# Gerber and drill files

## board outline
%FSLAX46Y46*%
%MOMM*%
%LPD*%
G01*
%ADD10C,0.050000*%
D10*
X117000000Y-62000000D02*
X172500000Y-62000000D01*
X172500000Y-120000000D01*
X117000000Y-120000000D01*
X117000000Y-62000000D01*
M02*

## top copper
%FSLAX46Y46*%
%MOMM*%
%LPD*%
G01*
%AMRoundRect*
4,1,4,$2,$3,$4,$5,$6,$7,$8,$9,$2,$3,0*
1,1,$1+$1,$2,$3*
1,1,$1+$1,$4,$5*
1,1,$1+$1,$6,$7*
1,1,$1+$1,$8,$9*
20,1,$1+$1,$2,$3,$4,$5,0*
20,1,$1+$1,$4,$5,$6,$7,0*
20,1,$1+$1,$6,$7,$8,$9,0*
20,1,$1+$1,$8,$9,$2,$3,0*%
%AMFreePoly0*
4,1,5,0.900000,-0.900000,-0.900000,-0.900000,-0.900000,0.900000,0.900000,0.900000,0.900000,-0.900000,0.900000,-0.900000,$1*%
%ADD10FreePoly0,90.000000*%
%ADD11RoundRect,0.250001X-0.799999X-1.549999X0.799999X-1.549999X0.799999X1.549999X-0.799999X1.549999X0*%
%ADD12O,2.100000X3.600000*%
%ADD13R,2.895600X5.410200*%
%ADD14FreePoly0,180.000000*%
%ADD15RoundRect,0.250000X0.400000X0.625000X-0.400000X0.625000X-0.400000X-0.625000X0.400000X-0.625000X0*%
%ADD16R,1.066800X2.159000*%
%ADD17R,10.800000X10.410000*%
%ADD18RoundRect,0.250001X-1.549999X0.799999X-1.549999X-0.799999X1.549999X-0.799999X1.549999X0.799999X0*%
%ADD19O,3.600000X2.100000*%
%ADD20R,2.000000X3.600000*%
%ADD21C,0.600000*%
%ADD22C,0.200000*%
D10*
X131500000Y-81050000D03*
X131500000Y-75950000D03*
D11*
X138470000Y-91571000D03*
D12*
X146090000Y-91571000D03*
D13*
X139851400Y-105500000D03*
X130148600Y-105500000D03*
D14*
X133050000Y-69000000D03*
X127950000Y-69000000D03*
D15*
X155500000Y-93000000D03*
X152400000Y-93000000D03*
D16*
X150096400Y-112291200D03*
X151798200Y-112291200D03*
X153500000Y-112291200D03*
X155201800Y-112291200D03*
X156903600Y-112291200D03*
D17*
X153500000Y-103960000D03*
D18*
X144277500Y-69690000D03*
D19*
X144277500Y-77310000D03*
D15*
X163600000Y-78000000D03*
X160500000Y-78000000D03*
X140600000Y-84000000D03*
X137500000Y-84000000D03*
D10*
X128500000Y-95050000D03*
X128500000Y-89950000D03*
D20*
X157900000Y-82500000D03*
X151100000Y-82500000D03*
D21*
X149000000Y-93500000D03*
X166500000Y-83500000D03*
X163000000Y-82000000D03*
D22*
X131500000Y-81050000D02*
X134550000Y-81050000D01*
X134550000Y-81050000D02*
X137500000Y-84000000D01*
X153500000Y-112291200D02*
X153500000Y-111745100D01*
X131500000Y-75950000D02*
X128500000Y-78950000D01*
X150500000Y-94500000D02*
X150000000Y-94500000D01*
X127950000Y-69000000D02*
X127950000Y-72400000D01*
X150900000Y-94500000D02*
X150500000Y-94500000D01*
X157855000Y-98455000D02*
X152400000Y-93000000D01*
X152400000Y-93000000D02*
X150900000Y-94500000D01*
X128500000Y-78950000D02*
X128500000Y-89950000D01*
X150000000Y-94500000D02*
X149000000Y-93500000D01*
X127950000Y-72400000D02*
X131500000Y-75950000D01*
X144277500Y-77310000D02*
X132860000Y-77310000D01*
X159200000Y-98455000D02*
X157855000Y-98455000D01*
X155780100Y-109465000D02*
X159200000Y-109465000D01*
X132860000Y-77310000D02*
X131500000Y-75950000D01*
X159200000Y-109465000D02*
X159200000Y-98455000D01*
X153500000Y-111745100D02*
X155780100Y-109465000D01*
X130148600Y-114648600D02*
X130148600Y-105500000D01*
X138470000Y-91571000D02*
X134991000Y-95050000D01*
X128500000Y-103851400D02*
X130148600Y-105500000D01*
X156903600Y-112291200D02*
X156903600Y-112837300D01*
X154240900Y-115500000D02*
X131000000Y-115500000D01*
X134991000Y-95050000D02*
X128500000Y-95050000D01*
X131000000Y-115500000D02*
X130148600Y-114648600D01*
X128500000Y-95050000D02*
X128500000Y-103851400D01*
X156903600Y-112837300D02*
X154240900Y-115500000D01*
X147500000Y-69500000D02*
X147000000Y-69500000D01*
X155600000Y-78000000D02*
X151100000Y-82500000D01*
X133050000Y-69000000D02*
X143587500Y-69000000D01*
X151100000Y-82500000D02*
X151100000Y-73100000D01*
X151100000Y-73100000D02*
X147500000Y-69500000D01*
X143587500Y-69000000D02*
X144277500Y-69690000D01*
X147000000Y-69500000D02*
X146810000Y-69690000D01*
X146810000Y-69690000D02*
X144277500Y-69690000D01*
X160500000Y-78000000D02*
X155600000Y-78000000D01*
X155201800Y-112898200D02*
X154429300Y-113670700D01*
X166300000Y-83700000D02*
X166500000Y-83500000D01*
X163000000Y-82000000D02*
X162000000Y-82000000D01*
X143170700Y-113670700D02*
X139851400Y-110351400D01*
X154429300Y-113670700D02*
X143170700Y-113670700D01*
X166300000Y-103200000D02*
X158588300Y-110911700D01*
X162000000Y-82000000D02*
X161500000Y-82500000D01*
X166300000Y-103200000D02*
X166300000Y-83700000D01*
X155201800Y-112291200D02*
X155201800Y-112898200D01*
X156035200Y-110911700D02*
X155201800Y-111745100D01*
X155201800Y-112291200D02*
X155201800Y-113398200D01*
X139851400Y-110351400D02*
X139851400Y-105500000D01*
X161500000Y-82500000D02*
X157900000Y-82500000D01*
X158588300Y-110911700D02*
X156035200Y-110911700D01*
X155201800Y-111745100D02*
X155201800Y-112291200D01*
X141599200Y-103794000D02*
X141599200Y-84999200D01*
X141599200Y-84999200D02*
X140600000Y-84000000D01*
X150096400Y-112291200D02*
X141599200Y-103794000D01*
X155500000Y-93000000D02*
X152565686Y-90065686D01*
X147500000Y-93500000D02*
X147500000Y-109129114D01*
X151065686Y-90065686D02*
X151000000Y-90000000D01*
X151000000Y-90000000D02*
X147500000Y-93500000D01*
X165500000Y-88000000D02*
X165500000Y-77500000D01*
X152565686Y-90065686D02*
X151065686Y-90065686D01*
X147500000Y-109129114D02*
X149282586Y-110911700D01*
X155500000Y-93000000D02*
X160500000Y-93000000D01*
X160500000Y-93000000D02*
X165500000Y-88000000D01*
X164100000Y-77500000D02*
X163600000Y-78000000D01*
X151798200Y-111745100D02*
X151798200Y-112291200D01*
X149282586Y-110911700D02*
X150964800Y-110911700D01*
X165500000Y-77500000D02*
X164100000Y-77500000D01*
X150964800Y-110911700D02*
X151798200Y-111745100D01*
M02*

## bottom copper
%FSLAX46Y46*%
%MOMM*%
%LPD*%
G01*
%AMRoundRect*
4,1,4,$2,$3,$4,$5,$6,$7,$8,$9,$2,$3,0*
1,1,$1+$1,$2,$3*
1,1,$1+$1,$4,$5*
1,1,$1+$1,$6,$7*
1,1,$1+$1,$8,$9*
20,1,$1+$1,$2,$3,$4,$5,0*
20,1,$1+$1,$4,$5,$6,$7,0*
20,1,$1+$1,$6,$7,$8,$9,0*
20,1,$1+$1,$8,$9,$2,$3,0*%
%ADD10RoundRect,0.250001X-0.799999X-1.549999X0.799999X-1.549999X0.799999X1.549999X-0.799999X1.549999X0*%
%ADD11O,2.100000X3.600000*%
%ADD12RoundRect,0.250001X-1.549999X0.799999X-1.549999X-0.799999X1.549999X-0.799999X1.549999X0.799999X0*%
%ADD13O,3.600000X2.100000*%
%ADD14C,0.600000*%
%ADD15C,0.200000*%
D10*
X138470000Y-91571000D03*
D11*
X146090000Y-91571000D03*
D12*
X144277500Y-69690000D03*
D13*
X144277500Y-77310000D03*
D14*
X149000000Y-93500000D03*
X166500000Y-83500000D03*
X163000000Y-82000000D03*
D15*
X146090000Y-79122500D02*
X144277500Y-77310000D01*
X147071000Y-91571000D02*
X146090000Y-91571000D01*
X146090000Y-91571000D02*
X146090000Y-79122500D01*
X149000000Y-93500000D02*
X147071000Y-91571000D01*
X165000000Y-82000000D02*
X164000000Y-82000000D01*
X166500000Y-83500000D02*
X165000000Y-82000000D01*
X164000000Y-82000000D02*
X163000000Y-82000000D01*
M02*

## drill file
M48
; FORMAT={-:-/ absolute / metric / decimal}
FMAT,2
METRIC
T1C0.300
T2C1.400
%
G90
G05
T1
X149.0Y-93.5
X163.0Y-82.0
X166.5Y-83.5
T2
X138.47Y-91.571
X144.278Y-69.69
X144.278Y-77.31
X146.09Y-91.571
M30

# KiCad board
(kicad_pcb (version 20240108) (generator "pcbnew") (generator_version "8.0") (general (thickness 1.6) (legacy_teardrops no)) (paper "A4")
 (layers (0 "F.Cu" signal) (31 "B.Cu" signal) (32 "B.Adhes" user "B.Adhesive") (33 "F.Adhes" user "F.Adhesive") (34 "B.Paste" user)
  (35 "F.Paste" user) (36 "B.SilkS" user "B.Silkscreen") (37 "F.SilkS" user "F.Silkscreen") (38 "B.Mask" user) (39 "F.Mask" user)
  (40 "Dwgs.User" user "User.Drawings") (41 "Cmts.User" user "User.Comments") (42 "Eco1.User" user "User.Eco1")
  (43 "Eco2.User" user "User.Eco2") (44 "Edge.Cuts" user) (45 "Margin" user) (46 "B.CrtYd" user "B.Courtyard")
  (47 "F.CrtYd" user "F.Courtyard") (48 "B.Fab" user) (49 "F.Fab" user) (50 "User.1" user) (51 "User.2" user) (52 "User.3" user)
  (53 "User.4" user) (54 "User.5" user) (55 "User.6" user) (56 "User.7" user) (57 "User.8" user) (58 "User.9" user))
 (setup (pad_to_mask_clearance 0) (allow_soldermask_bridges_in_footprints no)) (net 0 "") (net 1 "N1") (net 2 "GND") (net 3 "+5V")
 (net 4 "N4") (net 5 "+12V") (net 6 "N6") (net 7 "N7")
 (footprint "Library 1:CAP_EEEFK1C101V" (layer "F.Cu") (at 131.5 78.5 90)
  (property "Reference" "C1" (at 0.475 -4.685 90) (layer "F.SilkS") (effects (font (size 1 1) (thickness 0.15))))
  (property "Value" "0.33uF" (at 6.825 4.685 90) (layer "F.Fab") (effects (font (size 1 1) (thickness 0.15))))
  (pad "1" smd custom (at -2.55 0 90) (size 1.8 1.8) (layers "F.Cu") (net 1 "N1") (options (clearance outline) (anchor rect)) (primitives))
  (pad "2" smd custom (at 2.55 0 90) (size 1.8 1.8) (layers "F.Cu") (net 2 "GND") (options (clearance outline) (anchor rect)) (primitives)))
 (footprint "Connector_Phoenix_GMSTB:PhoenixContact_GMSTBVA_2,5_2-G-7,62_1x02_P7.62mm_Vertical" (layer "F.Cu") (at 138.47 91.571)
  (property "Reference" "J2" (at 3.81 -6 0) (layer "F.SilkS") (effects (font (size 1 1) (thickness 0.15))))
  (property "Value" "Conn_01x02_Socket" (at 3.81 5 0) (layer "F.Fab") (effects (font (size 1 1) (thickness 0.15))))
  (pad "1" thru_hole roundrect (at 0 0) (size 2.1 3.6) (drill 1.4) (layers "*.Cu" "*.Mask") (remove_unused_layers no)
   (roundrect_rratio 0.119048) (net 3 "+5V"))
  (pad "2" thru_hole oval (at 7.62 0) (size 2.1 3.6) (drill 1.4) (layers "*.Cu" "*.Mask") (remove_unused_layers no) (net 2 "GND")))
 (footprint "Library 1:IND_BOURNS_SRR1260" (layer "F.Cu") (at 135 105.5 180)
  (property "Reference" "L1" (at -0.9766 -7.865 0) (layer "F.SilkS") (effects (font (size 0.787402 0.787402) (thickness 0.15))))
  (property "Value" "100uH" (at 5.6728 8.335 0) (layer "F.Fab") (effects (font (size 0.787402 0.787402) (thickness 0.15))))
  (pad "1" smd rect (at -4.8514 0 180) (size 2.8956 5.4102) (layers "F.Cu" "F.Paste" "F.Mask") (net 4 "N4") (solder_mask_margin 0.102))
  (pad "2" smd rect (at 4.8514 0 180) (size 2.8956 5.4102) (layers "F.Cu" "F.Paste" "F.Mask") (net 3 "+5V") (solder_mask_margin 0.102)))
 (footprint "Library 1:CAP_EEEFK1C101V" (layer "F.Cu") (at 130.5 69 180)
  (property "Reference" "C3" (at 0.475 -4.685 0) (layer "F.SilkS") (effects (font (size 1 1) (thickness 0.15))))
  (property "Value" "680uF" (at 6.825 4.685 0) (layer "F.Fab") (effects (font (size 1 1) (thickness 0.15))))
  (pad "1" smd custom (at -2.55 0 180) (size 1.8 1.8) (layers "F.Cu") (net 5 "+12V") (options (clearance outline) (anchor rect))
   (primitives))
  (pad "2" smd custom (at 2.55 0 180) (size 1.8 1.8) (layers "F.Cu") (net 2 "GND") (options (clearance outline) (anchor rect)) (primitives)))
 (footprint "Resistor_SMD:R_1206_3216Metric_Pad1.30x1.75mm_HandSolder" (layer "F.Cu") (at 153.95 93 180)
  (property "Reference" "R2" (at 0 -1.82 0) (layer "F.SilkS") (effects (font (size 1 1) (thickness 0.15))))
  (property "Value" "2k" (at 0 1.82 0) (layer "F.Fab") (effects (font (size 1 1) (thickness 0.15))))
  (pad "1" smd roundrect (at -1.55 0 180) (size 1.3 1.75) (layers "F.Cu" "F.Paste" "F.Mask") (roundrect_rratio 0.192308) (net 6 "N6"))
  (pad "2" smd roundrect (at 1.55 0 180) (size 1.3 1.75) (layers "F.Cu" "F.Paste" "F.Mask") (roundrect_rratio 0.192308) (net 2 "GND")))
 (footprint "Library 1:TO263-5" (layer "F.Cu") (at 153.5 106.5)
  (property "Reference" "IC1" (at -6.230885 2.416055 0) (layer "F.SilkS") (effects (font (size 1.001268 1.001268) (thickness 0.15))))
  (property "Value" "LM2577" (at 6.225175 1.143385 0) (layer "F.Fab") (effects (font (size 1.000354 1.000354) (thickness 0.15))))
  (pad "1" smd rect (at -3.4036 5.7912) (size 1.0668 2.159) (layers "F.Cu" "F.Paste" "F.Mask") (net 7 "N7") (solder_mask_margin 0.102))
  (pad "2" smd rect (at -1.7018 5.7912) (size 1.0668 2.159) (layers "F.Cu" "F.Paste" "F.Mask") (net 6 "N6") (solder_mask_margin 0.102))
  (pad "3" smd rect (at 0 5.7912) (size 1.0668 2.159) (layers "F.Cu" "F.Paste" "F.Mask") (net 2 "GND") (solder_mask_margin 0.102))
  (pad "4" smd rect (at 1.7018 5.7912) (size 1.0668 2.159) (layers "F.Cu" "F.Paste" "F.Mask") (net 4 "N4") (solder_mask_margin 0.102))
  (pad "5" smd rect (at 3.4036 5.7912) (size 1.0668 2.159) (layers "F.Cu" "F.Paste" "F.Mask") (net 3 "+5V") (solder_mask_margin 0.102))
  (pad "6" smd rect (at 0 -2.54) (size 10.8 10.41) (layers "F.Cu" "F.Paste" "F.Mask") (solder_mask_margin 0.102)))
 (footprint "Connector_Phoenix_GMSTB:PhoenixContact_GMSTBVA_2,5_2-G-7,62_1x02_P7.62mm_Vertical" (layer "F.Cu") (at 144.2775 69.69 -90)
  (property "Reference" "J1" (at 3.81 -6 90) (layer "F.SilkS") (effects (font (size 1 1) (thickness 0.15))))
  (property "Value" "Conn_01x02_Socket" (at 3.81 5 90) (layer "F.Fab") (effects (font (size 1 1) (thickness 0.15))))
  (pad "1" thru_hole roundrect (at 0 0 270) (size 2.1 3.6) (drill 1.4) (layers "*.Cu" "*.Mask") (remove_unused_layers no)
   (roundrect_rratio 0.119048) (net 5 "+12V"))
  (pad "2" thru_hole oval (at 7.62 0 270) (size 2.1 3.6) (drill 1.4) (layers "*.Cu" "*.Mask") (remove_unused_layers no) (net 2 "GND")))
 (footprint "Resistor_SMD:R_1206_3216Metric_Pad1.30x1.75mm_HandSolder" (layer "F.Cu") (at 162.05 78 180)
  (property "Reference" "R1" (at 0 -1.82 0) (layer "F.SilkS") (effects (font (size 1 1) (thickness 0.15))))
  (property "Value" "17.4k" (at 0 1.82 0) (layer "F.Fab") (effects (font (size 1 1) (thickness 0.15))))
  (pad "1" smd roundrect (at -1.55 0 180) (size 1.3 1.75) (layers "F.Cu" "F.Paste" "F.Mask") (roundrect_rratio 0.192308) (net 6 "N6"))
  (pad "2" smd roundrect (at 1.55 0 180) (size 1.3 1.75) (layers "F.Cu" "F.Paste" "F.Mask") (roundrect_rratio 0.192308) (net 5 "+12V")))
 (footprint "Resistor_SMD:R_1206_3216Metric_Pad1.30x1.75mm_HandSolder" (layer "F.Cu") (at 139.05 84 180)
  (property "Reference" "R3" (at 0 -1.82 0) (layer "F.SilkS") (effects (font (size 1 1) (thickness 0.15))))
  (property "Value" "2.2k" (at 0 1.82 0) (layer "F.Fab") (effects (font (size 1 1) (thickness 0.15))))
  (pad "1" smd roundrect (at -1.55 0 180) (size 1.3 1.75) (layers "F.Cu" "F.Paste" "F.Mask") (roundrect_rratio 0.192308) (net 7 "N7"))
  (pad "2" smd roundrect (at 1.55 0 180) (size 1.3 1.75) (layers "F.Cu" "F.Paste" "F.Mask") (roundrect_rratio 0.192308) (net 1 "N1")))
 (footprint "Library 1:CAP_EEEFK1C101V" (layer "F.Cu") (at 128.5 92.5 90)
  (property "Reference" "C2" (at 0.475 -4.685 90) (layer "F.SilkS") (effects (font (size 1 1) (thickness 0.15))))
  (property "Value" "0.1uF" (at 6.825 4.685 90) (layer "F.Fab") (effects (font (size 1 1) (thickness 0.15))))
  (pad "1" smd custom (at -2.55 0 90) (size 1.8 1.8) (layers "F.Cu") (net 3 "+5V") (options (clearance outline) (anchor rect)) (primitives))
  (pad "2" smd custom (at 2.55 0 90) (size 1.8 1.8) (layers "F.Cu") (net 2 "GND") (options (clearance outline) (anchor rect)) (primitives)))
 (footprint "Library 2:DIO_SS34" (layer "F.Cu") (at 154.5 82.5)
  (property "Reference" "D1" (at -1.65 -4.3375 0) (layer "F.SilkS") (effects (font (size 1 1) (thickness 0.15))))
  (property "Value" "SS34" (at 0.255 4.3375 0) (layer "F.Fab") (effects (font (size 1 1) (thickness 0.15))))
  (pad "A" smd rect (at 3.4 0) (size 2 3.6) (layers "F.Cu" "F.Paste" "F.Mask") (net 4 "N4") (solder_mask_margin 0.102))
  (pad "C" smd rect (at -3.4 0) (size 2 3.6) (layers "F.Cu" "F.Paste" "F.Mask") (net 5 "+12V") (solder_mask_margin 0.102)))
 (gr_rect (start 117 62) (end 172.5 120) (stroke (width 0.05) (type default)) (fill none) (layer "Edge.Cuts"))
 (segment (start 131.5 81.05) (end 134.55 81.05) (width 0.2) (layer "F.Cu") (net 1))
 (segment (start 134.55 81.05) (end 137.5 84) (width 0.2) (layer "F.Cu") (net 1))
 (segment (start 153.5 112.2912) (end 153.5 111.7451) (width 0.2) (layer "F.Cu") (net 2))
 (segment (start 131.5 75.95) (end 128.5 78.95) (width 0.2) (layer "F.Cu") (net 2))
 (segment (start 150.5 94.5) (end 150 94.5) (width 0.2) (layer "F.Cu") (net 2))
 (segment (start 127.95 69) (end 127.95 72.4) (width 0.2) (layer "F.Cu") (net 2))
 (segment (start 150.9 94.5) (end 150.5 94.5) (width 0.2) (layer "F.Cu") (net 2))
 (segment (start 157.855 98.455) (end 152.4 93) (width 0.2) (layer "F.Cu") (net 2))
 (segment (start 152.4 93) (end 150.9 94.5) (width 0.2) (layer "F.Cu") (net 2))
 (segment (start 128.5 78.95) (end 128.5 89.95) (width 0.2) (layer "F.Cu") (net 2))
 (segment (start 150 94.5) (end 149 93.5) (width 0.2) (layer "F.Cu") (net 2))
 (segment (start 127.95 72.4) (end 131.5 75.95) (width 0.2) (layer "F.Cu") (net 2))
 (segment (start 144.2775 77.31) (end 132.86 77.31) (width 0.2) (layer "F.Cu") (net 2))
 (segment (start 159.2 98.455) (end 157.855 98.455) (width 0.2) (layer "F.Cu") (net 2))
 (segment (start 155.7801 109.465) (end 159.2 109.465) (width 0.2) (layer "F.Cu") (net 2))
 (segment (start 132.86 77.31) (end 131.5 75.95) (width 0.2) (layer "F.Cu") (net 2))
 (segment (start 159.2 109.465) (end 159.2 98.455) (width 0.2) (layer "F.Cu") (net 2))
 (segment (start 153.5 111.7451) (end 155.7801 109.465) (width 0.2) (layer "F.Cu") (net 2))
 (via (at 149 93.5) (size 0.6) (drill 0.3) (layers "F.Cu" "B.Cu") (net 2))
 (segment (start 146.09 79.1225) (end 144.2775 77.31) (width 0.2) (layer "B.Cu") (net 2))
 (segment (start 147.071 91.571) (end 146.09 91.571) (width 0.2) (layer "B.Cu") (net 2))
 (segment (start 146.09 91.571) (end 146.09 79.1225) (width 0.2) (layer "B.Cu") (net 2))
 (segment (start 149 93.5) (end 147.071 91.571) (width 0.2) (layer "B.Cu") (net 2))
 (segment (start 130.1486 114.6486) (end 130.1486 105.5) (width 0.2) (layer "F.Cu") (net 3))
 (segment (start 138.47 91.571) (end 134.991 95.05) (width 0.2) (layer "F.Cu") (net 3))
 (segment (start 128.5 103.8514) (end 130.1486 105.5) (width 0.2) (layer "F.Cu") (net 3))
 (segment (start 156.9036 112.2912) (end 156.9036 112.8373) (width 0.2) (layer "F.Cu") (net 3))
 (segment (start 154.2409 115.5) (end 131 115.5) (width 0.2) (layer "F.Cu") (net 3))
 (segment (start 134.991 95.05) (end 128.5 95.05) (width 0.2) (layer "F.Cu") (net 3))
 (segment (start 131 115.5) (end 130.1486 114.6486) (width 0.2) (layer "F.Cu") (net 3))
 (segment (start 128.5 95.05) (end 128.5 103.8514) (width 0.2) (layer "F.Cu") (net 3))
 (segment (start 156.9036 112.8373) (end 154.2409 115.5) (width 0.2) (layer "F.Cu") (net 3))
 (segment (start 147.5 69.5) (end 147 69.5) (width 0.2) (layer "F.Cu") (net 5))
 (segment (start 155.6 78) (end 151.1 82.5) (width 0.2) (layer "F.Cu") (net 5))
 (segment (start 133.05 69) (end 143.5875 69) (width 0.2) (layer "F.Cu") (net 5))
 (segment (start 151.1 82.5) (end 151.1 73.1) (width 0.2) (layer "F.Cu") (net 5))
 (segment (start 151.1 73.1) (end 147.5 69.5) (width 0.2) (layer "F.Cu") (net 5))
 (segment (start 143.5875 69) (end 144.2775 69.69) (width 0.2) (layer "F.Cu") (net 5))
 (segment (start 147 69.5) (end 146.81 69.69) (width 0.2) (layer "F.Cu") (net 5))
 (segment (start 146.81 69.69) (end 144.2775 69.69) (width 0.2) (layer "F.Cu") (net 5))
 (segment (start 160.5 78) (end 155.6 78) (width 0.2) (layer "F.Cu") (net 5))
 (segment (start 155.2018 112.8982) (end 154.4293 113.6707) (width 0.2) (layer "F.Cu") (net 4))
 (segment (start 166.3 83.7) (end 166.5 83.5) (width 0.2) (layer "F.Cu") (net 4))
 (segment (start 163 82) (end 162 82) (width 0.2) (layer "F.Cu") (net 4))
 (segment (start 143.1707 113.6707) (end 139.8514 110.3514) (width 0.2) (layer "F.Cu") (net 4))
 (segment (start 154.4293 113.6707) (end 143.1707 113.6707) (width 0.2) (layer "F.Cu") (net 4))
 (segment (start 166.3 103.2) (end 158.5883 110.9117) (width 0.2) (layer "F.Cu") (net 4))
 (segment (start 162 82) (end 161.5 82.5) (width 0.2) (layer "F.Cu") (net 4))
 (segment (start 166.3 103.2) (end 166.3 83.7) (width 0.2) (layer "F.Cu") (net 4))
 (segment (start 155.2018 112.2912) (end 155.2018 112.8982) (width 0.2) (layer "F.Cu") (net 4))
 (segment (start 156.0352 110.9117) (end 155.2018 111.7451) (width 0.2) (layer "F.Cu") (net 4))
 (segment (start 155.2018 112.2912) (end 155.2018 113.3982) (width 0.2) (layer "F.Cu") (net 4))
 (segment (start 139.8514 110.3514) (end 139.8514 105.5) (width 0.2) (layer "F.Cu") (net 4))
 (segment (start 161.5 82.5) (end 157.9 82.5) (width 0.2) (layer "F.Cu") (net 4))
 (segment (start 158.5883 110.9117) (end 156.0352 110.9117) (width 0.2) (layer "F.Cu") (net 4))
 (segment (start 155.2018 111.7451) (end 155.2018 112.2912) (width 0.2) (layer "F.Cu") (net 4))
 (via (at 166.5 83.5) (size 0.6) (drill 0.3) (layers "F.Cu" "B.Cu") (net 4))
 (via (at 163 82) (size 0.6) (drill 0.3) (layers "F.Cu" "B.Cu") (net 4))
 (segment (start 165 82) (end 164 82) (width 0.2) (layer "B.Cu") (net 4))
 (segment (start 166.5 83.5) (end 165 82) (width 0.2) (layer "B.Cu") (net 4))
 (segment (start 164 82) (end 163 82) (width 0.2) (layer "B.Cu") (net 4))
 (segment (start 141.5992 103.794) (end 141.5992 84.9992) (width 0.2) (layer "F.Cu") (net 7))
 (segment (start 141.5992 84.9992) (end 140.6 84) (width 0.2) (layer "F.Cu") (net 7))
 (segment (start 150.0964 112.2912) (end 141.5992 103.794) (width 0.2) (layer "F.Cu") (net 7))
 (segment (start 155.5 93) (end 152.565686 90.065686) (width 0.2) (layer "F.Cu") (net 6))
 (segment (start 147.5 93.5) (end 147.5 109.129114) (width 0.2) (layer "F.Cu") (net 6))
 (segment (start 151.065686 90.065686) (end 151 90) (width 0.2) (layer "F.Cu") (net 6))
 (segment (start 151 90) (end 147.5 93.5) (width 0.2) (layer "F.Cu") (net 6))
 (segment (start 165.5 88) (end 165.5 77.5) (width 0.2) (layer "F.Cu") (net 6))
 (segment (start 152.565686 90.065686) (end 151.065686 90.065686) (width 0.2) (layer "F.Cu") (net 6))
 (segment (start 147.5 109.129114) (end 149.282586 110.9117) (width 0.2) (layer "F.Cu") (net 6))
 (segment (start 155.5 93) (end 160.5 93) (width 0.2) (layer "F.Cu") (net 6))
 (segment (start 160.5 93) (end 165.5 88) (width 0.2) (layer "F.Cu") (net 6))
 (segment (start 164.1 77.5) (end 163.6 78) (width 0.2) (layer "F.Cu") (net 6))
 (segment (start 151.7982 111.7451) (end 151.7982 112.2912) (width 0.2) (layer "F.Cu") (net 6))
 (segment (start 149.282586 110.9117) (end 150.9648 110.9117) (width 0.2) (layer "F.Cu") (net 6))
 (segment (start 165.5 77.5) (end 164.1 77.5) (width 0.2) (layer "F.Cu") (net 6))
 (segment (start 150.9648 110.9117) (end 151.7982 111.7451) (width 0.2) (layer "F.Cu") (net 6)))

